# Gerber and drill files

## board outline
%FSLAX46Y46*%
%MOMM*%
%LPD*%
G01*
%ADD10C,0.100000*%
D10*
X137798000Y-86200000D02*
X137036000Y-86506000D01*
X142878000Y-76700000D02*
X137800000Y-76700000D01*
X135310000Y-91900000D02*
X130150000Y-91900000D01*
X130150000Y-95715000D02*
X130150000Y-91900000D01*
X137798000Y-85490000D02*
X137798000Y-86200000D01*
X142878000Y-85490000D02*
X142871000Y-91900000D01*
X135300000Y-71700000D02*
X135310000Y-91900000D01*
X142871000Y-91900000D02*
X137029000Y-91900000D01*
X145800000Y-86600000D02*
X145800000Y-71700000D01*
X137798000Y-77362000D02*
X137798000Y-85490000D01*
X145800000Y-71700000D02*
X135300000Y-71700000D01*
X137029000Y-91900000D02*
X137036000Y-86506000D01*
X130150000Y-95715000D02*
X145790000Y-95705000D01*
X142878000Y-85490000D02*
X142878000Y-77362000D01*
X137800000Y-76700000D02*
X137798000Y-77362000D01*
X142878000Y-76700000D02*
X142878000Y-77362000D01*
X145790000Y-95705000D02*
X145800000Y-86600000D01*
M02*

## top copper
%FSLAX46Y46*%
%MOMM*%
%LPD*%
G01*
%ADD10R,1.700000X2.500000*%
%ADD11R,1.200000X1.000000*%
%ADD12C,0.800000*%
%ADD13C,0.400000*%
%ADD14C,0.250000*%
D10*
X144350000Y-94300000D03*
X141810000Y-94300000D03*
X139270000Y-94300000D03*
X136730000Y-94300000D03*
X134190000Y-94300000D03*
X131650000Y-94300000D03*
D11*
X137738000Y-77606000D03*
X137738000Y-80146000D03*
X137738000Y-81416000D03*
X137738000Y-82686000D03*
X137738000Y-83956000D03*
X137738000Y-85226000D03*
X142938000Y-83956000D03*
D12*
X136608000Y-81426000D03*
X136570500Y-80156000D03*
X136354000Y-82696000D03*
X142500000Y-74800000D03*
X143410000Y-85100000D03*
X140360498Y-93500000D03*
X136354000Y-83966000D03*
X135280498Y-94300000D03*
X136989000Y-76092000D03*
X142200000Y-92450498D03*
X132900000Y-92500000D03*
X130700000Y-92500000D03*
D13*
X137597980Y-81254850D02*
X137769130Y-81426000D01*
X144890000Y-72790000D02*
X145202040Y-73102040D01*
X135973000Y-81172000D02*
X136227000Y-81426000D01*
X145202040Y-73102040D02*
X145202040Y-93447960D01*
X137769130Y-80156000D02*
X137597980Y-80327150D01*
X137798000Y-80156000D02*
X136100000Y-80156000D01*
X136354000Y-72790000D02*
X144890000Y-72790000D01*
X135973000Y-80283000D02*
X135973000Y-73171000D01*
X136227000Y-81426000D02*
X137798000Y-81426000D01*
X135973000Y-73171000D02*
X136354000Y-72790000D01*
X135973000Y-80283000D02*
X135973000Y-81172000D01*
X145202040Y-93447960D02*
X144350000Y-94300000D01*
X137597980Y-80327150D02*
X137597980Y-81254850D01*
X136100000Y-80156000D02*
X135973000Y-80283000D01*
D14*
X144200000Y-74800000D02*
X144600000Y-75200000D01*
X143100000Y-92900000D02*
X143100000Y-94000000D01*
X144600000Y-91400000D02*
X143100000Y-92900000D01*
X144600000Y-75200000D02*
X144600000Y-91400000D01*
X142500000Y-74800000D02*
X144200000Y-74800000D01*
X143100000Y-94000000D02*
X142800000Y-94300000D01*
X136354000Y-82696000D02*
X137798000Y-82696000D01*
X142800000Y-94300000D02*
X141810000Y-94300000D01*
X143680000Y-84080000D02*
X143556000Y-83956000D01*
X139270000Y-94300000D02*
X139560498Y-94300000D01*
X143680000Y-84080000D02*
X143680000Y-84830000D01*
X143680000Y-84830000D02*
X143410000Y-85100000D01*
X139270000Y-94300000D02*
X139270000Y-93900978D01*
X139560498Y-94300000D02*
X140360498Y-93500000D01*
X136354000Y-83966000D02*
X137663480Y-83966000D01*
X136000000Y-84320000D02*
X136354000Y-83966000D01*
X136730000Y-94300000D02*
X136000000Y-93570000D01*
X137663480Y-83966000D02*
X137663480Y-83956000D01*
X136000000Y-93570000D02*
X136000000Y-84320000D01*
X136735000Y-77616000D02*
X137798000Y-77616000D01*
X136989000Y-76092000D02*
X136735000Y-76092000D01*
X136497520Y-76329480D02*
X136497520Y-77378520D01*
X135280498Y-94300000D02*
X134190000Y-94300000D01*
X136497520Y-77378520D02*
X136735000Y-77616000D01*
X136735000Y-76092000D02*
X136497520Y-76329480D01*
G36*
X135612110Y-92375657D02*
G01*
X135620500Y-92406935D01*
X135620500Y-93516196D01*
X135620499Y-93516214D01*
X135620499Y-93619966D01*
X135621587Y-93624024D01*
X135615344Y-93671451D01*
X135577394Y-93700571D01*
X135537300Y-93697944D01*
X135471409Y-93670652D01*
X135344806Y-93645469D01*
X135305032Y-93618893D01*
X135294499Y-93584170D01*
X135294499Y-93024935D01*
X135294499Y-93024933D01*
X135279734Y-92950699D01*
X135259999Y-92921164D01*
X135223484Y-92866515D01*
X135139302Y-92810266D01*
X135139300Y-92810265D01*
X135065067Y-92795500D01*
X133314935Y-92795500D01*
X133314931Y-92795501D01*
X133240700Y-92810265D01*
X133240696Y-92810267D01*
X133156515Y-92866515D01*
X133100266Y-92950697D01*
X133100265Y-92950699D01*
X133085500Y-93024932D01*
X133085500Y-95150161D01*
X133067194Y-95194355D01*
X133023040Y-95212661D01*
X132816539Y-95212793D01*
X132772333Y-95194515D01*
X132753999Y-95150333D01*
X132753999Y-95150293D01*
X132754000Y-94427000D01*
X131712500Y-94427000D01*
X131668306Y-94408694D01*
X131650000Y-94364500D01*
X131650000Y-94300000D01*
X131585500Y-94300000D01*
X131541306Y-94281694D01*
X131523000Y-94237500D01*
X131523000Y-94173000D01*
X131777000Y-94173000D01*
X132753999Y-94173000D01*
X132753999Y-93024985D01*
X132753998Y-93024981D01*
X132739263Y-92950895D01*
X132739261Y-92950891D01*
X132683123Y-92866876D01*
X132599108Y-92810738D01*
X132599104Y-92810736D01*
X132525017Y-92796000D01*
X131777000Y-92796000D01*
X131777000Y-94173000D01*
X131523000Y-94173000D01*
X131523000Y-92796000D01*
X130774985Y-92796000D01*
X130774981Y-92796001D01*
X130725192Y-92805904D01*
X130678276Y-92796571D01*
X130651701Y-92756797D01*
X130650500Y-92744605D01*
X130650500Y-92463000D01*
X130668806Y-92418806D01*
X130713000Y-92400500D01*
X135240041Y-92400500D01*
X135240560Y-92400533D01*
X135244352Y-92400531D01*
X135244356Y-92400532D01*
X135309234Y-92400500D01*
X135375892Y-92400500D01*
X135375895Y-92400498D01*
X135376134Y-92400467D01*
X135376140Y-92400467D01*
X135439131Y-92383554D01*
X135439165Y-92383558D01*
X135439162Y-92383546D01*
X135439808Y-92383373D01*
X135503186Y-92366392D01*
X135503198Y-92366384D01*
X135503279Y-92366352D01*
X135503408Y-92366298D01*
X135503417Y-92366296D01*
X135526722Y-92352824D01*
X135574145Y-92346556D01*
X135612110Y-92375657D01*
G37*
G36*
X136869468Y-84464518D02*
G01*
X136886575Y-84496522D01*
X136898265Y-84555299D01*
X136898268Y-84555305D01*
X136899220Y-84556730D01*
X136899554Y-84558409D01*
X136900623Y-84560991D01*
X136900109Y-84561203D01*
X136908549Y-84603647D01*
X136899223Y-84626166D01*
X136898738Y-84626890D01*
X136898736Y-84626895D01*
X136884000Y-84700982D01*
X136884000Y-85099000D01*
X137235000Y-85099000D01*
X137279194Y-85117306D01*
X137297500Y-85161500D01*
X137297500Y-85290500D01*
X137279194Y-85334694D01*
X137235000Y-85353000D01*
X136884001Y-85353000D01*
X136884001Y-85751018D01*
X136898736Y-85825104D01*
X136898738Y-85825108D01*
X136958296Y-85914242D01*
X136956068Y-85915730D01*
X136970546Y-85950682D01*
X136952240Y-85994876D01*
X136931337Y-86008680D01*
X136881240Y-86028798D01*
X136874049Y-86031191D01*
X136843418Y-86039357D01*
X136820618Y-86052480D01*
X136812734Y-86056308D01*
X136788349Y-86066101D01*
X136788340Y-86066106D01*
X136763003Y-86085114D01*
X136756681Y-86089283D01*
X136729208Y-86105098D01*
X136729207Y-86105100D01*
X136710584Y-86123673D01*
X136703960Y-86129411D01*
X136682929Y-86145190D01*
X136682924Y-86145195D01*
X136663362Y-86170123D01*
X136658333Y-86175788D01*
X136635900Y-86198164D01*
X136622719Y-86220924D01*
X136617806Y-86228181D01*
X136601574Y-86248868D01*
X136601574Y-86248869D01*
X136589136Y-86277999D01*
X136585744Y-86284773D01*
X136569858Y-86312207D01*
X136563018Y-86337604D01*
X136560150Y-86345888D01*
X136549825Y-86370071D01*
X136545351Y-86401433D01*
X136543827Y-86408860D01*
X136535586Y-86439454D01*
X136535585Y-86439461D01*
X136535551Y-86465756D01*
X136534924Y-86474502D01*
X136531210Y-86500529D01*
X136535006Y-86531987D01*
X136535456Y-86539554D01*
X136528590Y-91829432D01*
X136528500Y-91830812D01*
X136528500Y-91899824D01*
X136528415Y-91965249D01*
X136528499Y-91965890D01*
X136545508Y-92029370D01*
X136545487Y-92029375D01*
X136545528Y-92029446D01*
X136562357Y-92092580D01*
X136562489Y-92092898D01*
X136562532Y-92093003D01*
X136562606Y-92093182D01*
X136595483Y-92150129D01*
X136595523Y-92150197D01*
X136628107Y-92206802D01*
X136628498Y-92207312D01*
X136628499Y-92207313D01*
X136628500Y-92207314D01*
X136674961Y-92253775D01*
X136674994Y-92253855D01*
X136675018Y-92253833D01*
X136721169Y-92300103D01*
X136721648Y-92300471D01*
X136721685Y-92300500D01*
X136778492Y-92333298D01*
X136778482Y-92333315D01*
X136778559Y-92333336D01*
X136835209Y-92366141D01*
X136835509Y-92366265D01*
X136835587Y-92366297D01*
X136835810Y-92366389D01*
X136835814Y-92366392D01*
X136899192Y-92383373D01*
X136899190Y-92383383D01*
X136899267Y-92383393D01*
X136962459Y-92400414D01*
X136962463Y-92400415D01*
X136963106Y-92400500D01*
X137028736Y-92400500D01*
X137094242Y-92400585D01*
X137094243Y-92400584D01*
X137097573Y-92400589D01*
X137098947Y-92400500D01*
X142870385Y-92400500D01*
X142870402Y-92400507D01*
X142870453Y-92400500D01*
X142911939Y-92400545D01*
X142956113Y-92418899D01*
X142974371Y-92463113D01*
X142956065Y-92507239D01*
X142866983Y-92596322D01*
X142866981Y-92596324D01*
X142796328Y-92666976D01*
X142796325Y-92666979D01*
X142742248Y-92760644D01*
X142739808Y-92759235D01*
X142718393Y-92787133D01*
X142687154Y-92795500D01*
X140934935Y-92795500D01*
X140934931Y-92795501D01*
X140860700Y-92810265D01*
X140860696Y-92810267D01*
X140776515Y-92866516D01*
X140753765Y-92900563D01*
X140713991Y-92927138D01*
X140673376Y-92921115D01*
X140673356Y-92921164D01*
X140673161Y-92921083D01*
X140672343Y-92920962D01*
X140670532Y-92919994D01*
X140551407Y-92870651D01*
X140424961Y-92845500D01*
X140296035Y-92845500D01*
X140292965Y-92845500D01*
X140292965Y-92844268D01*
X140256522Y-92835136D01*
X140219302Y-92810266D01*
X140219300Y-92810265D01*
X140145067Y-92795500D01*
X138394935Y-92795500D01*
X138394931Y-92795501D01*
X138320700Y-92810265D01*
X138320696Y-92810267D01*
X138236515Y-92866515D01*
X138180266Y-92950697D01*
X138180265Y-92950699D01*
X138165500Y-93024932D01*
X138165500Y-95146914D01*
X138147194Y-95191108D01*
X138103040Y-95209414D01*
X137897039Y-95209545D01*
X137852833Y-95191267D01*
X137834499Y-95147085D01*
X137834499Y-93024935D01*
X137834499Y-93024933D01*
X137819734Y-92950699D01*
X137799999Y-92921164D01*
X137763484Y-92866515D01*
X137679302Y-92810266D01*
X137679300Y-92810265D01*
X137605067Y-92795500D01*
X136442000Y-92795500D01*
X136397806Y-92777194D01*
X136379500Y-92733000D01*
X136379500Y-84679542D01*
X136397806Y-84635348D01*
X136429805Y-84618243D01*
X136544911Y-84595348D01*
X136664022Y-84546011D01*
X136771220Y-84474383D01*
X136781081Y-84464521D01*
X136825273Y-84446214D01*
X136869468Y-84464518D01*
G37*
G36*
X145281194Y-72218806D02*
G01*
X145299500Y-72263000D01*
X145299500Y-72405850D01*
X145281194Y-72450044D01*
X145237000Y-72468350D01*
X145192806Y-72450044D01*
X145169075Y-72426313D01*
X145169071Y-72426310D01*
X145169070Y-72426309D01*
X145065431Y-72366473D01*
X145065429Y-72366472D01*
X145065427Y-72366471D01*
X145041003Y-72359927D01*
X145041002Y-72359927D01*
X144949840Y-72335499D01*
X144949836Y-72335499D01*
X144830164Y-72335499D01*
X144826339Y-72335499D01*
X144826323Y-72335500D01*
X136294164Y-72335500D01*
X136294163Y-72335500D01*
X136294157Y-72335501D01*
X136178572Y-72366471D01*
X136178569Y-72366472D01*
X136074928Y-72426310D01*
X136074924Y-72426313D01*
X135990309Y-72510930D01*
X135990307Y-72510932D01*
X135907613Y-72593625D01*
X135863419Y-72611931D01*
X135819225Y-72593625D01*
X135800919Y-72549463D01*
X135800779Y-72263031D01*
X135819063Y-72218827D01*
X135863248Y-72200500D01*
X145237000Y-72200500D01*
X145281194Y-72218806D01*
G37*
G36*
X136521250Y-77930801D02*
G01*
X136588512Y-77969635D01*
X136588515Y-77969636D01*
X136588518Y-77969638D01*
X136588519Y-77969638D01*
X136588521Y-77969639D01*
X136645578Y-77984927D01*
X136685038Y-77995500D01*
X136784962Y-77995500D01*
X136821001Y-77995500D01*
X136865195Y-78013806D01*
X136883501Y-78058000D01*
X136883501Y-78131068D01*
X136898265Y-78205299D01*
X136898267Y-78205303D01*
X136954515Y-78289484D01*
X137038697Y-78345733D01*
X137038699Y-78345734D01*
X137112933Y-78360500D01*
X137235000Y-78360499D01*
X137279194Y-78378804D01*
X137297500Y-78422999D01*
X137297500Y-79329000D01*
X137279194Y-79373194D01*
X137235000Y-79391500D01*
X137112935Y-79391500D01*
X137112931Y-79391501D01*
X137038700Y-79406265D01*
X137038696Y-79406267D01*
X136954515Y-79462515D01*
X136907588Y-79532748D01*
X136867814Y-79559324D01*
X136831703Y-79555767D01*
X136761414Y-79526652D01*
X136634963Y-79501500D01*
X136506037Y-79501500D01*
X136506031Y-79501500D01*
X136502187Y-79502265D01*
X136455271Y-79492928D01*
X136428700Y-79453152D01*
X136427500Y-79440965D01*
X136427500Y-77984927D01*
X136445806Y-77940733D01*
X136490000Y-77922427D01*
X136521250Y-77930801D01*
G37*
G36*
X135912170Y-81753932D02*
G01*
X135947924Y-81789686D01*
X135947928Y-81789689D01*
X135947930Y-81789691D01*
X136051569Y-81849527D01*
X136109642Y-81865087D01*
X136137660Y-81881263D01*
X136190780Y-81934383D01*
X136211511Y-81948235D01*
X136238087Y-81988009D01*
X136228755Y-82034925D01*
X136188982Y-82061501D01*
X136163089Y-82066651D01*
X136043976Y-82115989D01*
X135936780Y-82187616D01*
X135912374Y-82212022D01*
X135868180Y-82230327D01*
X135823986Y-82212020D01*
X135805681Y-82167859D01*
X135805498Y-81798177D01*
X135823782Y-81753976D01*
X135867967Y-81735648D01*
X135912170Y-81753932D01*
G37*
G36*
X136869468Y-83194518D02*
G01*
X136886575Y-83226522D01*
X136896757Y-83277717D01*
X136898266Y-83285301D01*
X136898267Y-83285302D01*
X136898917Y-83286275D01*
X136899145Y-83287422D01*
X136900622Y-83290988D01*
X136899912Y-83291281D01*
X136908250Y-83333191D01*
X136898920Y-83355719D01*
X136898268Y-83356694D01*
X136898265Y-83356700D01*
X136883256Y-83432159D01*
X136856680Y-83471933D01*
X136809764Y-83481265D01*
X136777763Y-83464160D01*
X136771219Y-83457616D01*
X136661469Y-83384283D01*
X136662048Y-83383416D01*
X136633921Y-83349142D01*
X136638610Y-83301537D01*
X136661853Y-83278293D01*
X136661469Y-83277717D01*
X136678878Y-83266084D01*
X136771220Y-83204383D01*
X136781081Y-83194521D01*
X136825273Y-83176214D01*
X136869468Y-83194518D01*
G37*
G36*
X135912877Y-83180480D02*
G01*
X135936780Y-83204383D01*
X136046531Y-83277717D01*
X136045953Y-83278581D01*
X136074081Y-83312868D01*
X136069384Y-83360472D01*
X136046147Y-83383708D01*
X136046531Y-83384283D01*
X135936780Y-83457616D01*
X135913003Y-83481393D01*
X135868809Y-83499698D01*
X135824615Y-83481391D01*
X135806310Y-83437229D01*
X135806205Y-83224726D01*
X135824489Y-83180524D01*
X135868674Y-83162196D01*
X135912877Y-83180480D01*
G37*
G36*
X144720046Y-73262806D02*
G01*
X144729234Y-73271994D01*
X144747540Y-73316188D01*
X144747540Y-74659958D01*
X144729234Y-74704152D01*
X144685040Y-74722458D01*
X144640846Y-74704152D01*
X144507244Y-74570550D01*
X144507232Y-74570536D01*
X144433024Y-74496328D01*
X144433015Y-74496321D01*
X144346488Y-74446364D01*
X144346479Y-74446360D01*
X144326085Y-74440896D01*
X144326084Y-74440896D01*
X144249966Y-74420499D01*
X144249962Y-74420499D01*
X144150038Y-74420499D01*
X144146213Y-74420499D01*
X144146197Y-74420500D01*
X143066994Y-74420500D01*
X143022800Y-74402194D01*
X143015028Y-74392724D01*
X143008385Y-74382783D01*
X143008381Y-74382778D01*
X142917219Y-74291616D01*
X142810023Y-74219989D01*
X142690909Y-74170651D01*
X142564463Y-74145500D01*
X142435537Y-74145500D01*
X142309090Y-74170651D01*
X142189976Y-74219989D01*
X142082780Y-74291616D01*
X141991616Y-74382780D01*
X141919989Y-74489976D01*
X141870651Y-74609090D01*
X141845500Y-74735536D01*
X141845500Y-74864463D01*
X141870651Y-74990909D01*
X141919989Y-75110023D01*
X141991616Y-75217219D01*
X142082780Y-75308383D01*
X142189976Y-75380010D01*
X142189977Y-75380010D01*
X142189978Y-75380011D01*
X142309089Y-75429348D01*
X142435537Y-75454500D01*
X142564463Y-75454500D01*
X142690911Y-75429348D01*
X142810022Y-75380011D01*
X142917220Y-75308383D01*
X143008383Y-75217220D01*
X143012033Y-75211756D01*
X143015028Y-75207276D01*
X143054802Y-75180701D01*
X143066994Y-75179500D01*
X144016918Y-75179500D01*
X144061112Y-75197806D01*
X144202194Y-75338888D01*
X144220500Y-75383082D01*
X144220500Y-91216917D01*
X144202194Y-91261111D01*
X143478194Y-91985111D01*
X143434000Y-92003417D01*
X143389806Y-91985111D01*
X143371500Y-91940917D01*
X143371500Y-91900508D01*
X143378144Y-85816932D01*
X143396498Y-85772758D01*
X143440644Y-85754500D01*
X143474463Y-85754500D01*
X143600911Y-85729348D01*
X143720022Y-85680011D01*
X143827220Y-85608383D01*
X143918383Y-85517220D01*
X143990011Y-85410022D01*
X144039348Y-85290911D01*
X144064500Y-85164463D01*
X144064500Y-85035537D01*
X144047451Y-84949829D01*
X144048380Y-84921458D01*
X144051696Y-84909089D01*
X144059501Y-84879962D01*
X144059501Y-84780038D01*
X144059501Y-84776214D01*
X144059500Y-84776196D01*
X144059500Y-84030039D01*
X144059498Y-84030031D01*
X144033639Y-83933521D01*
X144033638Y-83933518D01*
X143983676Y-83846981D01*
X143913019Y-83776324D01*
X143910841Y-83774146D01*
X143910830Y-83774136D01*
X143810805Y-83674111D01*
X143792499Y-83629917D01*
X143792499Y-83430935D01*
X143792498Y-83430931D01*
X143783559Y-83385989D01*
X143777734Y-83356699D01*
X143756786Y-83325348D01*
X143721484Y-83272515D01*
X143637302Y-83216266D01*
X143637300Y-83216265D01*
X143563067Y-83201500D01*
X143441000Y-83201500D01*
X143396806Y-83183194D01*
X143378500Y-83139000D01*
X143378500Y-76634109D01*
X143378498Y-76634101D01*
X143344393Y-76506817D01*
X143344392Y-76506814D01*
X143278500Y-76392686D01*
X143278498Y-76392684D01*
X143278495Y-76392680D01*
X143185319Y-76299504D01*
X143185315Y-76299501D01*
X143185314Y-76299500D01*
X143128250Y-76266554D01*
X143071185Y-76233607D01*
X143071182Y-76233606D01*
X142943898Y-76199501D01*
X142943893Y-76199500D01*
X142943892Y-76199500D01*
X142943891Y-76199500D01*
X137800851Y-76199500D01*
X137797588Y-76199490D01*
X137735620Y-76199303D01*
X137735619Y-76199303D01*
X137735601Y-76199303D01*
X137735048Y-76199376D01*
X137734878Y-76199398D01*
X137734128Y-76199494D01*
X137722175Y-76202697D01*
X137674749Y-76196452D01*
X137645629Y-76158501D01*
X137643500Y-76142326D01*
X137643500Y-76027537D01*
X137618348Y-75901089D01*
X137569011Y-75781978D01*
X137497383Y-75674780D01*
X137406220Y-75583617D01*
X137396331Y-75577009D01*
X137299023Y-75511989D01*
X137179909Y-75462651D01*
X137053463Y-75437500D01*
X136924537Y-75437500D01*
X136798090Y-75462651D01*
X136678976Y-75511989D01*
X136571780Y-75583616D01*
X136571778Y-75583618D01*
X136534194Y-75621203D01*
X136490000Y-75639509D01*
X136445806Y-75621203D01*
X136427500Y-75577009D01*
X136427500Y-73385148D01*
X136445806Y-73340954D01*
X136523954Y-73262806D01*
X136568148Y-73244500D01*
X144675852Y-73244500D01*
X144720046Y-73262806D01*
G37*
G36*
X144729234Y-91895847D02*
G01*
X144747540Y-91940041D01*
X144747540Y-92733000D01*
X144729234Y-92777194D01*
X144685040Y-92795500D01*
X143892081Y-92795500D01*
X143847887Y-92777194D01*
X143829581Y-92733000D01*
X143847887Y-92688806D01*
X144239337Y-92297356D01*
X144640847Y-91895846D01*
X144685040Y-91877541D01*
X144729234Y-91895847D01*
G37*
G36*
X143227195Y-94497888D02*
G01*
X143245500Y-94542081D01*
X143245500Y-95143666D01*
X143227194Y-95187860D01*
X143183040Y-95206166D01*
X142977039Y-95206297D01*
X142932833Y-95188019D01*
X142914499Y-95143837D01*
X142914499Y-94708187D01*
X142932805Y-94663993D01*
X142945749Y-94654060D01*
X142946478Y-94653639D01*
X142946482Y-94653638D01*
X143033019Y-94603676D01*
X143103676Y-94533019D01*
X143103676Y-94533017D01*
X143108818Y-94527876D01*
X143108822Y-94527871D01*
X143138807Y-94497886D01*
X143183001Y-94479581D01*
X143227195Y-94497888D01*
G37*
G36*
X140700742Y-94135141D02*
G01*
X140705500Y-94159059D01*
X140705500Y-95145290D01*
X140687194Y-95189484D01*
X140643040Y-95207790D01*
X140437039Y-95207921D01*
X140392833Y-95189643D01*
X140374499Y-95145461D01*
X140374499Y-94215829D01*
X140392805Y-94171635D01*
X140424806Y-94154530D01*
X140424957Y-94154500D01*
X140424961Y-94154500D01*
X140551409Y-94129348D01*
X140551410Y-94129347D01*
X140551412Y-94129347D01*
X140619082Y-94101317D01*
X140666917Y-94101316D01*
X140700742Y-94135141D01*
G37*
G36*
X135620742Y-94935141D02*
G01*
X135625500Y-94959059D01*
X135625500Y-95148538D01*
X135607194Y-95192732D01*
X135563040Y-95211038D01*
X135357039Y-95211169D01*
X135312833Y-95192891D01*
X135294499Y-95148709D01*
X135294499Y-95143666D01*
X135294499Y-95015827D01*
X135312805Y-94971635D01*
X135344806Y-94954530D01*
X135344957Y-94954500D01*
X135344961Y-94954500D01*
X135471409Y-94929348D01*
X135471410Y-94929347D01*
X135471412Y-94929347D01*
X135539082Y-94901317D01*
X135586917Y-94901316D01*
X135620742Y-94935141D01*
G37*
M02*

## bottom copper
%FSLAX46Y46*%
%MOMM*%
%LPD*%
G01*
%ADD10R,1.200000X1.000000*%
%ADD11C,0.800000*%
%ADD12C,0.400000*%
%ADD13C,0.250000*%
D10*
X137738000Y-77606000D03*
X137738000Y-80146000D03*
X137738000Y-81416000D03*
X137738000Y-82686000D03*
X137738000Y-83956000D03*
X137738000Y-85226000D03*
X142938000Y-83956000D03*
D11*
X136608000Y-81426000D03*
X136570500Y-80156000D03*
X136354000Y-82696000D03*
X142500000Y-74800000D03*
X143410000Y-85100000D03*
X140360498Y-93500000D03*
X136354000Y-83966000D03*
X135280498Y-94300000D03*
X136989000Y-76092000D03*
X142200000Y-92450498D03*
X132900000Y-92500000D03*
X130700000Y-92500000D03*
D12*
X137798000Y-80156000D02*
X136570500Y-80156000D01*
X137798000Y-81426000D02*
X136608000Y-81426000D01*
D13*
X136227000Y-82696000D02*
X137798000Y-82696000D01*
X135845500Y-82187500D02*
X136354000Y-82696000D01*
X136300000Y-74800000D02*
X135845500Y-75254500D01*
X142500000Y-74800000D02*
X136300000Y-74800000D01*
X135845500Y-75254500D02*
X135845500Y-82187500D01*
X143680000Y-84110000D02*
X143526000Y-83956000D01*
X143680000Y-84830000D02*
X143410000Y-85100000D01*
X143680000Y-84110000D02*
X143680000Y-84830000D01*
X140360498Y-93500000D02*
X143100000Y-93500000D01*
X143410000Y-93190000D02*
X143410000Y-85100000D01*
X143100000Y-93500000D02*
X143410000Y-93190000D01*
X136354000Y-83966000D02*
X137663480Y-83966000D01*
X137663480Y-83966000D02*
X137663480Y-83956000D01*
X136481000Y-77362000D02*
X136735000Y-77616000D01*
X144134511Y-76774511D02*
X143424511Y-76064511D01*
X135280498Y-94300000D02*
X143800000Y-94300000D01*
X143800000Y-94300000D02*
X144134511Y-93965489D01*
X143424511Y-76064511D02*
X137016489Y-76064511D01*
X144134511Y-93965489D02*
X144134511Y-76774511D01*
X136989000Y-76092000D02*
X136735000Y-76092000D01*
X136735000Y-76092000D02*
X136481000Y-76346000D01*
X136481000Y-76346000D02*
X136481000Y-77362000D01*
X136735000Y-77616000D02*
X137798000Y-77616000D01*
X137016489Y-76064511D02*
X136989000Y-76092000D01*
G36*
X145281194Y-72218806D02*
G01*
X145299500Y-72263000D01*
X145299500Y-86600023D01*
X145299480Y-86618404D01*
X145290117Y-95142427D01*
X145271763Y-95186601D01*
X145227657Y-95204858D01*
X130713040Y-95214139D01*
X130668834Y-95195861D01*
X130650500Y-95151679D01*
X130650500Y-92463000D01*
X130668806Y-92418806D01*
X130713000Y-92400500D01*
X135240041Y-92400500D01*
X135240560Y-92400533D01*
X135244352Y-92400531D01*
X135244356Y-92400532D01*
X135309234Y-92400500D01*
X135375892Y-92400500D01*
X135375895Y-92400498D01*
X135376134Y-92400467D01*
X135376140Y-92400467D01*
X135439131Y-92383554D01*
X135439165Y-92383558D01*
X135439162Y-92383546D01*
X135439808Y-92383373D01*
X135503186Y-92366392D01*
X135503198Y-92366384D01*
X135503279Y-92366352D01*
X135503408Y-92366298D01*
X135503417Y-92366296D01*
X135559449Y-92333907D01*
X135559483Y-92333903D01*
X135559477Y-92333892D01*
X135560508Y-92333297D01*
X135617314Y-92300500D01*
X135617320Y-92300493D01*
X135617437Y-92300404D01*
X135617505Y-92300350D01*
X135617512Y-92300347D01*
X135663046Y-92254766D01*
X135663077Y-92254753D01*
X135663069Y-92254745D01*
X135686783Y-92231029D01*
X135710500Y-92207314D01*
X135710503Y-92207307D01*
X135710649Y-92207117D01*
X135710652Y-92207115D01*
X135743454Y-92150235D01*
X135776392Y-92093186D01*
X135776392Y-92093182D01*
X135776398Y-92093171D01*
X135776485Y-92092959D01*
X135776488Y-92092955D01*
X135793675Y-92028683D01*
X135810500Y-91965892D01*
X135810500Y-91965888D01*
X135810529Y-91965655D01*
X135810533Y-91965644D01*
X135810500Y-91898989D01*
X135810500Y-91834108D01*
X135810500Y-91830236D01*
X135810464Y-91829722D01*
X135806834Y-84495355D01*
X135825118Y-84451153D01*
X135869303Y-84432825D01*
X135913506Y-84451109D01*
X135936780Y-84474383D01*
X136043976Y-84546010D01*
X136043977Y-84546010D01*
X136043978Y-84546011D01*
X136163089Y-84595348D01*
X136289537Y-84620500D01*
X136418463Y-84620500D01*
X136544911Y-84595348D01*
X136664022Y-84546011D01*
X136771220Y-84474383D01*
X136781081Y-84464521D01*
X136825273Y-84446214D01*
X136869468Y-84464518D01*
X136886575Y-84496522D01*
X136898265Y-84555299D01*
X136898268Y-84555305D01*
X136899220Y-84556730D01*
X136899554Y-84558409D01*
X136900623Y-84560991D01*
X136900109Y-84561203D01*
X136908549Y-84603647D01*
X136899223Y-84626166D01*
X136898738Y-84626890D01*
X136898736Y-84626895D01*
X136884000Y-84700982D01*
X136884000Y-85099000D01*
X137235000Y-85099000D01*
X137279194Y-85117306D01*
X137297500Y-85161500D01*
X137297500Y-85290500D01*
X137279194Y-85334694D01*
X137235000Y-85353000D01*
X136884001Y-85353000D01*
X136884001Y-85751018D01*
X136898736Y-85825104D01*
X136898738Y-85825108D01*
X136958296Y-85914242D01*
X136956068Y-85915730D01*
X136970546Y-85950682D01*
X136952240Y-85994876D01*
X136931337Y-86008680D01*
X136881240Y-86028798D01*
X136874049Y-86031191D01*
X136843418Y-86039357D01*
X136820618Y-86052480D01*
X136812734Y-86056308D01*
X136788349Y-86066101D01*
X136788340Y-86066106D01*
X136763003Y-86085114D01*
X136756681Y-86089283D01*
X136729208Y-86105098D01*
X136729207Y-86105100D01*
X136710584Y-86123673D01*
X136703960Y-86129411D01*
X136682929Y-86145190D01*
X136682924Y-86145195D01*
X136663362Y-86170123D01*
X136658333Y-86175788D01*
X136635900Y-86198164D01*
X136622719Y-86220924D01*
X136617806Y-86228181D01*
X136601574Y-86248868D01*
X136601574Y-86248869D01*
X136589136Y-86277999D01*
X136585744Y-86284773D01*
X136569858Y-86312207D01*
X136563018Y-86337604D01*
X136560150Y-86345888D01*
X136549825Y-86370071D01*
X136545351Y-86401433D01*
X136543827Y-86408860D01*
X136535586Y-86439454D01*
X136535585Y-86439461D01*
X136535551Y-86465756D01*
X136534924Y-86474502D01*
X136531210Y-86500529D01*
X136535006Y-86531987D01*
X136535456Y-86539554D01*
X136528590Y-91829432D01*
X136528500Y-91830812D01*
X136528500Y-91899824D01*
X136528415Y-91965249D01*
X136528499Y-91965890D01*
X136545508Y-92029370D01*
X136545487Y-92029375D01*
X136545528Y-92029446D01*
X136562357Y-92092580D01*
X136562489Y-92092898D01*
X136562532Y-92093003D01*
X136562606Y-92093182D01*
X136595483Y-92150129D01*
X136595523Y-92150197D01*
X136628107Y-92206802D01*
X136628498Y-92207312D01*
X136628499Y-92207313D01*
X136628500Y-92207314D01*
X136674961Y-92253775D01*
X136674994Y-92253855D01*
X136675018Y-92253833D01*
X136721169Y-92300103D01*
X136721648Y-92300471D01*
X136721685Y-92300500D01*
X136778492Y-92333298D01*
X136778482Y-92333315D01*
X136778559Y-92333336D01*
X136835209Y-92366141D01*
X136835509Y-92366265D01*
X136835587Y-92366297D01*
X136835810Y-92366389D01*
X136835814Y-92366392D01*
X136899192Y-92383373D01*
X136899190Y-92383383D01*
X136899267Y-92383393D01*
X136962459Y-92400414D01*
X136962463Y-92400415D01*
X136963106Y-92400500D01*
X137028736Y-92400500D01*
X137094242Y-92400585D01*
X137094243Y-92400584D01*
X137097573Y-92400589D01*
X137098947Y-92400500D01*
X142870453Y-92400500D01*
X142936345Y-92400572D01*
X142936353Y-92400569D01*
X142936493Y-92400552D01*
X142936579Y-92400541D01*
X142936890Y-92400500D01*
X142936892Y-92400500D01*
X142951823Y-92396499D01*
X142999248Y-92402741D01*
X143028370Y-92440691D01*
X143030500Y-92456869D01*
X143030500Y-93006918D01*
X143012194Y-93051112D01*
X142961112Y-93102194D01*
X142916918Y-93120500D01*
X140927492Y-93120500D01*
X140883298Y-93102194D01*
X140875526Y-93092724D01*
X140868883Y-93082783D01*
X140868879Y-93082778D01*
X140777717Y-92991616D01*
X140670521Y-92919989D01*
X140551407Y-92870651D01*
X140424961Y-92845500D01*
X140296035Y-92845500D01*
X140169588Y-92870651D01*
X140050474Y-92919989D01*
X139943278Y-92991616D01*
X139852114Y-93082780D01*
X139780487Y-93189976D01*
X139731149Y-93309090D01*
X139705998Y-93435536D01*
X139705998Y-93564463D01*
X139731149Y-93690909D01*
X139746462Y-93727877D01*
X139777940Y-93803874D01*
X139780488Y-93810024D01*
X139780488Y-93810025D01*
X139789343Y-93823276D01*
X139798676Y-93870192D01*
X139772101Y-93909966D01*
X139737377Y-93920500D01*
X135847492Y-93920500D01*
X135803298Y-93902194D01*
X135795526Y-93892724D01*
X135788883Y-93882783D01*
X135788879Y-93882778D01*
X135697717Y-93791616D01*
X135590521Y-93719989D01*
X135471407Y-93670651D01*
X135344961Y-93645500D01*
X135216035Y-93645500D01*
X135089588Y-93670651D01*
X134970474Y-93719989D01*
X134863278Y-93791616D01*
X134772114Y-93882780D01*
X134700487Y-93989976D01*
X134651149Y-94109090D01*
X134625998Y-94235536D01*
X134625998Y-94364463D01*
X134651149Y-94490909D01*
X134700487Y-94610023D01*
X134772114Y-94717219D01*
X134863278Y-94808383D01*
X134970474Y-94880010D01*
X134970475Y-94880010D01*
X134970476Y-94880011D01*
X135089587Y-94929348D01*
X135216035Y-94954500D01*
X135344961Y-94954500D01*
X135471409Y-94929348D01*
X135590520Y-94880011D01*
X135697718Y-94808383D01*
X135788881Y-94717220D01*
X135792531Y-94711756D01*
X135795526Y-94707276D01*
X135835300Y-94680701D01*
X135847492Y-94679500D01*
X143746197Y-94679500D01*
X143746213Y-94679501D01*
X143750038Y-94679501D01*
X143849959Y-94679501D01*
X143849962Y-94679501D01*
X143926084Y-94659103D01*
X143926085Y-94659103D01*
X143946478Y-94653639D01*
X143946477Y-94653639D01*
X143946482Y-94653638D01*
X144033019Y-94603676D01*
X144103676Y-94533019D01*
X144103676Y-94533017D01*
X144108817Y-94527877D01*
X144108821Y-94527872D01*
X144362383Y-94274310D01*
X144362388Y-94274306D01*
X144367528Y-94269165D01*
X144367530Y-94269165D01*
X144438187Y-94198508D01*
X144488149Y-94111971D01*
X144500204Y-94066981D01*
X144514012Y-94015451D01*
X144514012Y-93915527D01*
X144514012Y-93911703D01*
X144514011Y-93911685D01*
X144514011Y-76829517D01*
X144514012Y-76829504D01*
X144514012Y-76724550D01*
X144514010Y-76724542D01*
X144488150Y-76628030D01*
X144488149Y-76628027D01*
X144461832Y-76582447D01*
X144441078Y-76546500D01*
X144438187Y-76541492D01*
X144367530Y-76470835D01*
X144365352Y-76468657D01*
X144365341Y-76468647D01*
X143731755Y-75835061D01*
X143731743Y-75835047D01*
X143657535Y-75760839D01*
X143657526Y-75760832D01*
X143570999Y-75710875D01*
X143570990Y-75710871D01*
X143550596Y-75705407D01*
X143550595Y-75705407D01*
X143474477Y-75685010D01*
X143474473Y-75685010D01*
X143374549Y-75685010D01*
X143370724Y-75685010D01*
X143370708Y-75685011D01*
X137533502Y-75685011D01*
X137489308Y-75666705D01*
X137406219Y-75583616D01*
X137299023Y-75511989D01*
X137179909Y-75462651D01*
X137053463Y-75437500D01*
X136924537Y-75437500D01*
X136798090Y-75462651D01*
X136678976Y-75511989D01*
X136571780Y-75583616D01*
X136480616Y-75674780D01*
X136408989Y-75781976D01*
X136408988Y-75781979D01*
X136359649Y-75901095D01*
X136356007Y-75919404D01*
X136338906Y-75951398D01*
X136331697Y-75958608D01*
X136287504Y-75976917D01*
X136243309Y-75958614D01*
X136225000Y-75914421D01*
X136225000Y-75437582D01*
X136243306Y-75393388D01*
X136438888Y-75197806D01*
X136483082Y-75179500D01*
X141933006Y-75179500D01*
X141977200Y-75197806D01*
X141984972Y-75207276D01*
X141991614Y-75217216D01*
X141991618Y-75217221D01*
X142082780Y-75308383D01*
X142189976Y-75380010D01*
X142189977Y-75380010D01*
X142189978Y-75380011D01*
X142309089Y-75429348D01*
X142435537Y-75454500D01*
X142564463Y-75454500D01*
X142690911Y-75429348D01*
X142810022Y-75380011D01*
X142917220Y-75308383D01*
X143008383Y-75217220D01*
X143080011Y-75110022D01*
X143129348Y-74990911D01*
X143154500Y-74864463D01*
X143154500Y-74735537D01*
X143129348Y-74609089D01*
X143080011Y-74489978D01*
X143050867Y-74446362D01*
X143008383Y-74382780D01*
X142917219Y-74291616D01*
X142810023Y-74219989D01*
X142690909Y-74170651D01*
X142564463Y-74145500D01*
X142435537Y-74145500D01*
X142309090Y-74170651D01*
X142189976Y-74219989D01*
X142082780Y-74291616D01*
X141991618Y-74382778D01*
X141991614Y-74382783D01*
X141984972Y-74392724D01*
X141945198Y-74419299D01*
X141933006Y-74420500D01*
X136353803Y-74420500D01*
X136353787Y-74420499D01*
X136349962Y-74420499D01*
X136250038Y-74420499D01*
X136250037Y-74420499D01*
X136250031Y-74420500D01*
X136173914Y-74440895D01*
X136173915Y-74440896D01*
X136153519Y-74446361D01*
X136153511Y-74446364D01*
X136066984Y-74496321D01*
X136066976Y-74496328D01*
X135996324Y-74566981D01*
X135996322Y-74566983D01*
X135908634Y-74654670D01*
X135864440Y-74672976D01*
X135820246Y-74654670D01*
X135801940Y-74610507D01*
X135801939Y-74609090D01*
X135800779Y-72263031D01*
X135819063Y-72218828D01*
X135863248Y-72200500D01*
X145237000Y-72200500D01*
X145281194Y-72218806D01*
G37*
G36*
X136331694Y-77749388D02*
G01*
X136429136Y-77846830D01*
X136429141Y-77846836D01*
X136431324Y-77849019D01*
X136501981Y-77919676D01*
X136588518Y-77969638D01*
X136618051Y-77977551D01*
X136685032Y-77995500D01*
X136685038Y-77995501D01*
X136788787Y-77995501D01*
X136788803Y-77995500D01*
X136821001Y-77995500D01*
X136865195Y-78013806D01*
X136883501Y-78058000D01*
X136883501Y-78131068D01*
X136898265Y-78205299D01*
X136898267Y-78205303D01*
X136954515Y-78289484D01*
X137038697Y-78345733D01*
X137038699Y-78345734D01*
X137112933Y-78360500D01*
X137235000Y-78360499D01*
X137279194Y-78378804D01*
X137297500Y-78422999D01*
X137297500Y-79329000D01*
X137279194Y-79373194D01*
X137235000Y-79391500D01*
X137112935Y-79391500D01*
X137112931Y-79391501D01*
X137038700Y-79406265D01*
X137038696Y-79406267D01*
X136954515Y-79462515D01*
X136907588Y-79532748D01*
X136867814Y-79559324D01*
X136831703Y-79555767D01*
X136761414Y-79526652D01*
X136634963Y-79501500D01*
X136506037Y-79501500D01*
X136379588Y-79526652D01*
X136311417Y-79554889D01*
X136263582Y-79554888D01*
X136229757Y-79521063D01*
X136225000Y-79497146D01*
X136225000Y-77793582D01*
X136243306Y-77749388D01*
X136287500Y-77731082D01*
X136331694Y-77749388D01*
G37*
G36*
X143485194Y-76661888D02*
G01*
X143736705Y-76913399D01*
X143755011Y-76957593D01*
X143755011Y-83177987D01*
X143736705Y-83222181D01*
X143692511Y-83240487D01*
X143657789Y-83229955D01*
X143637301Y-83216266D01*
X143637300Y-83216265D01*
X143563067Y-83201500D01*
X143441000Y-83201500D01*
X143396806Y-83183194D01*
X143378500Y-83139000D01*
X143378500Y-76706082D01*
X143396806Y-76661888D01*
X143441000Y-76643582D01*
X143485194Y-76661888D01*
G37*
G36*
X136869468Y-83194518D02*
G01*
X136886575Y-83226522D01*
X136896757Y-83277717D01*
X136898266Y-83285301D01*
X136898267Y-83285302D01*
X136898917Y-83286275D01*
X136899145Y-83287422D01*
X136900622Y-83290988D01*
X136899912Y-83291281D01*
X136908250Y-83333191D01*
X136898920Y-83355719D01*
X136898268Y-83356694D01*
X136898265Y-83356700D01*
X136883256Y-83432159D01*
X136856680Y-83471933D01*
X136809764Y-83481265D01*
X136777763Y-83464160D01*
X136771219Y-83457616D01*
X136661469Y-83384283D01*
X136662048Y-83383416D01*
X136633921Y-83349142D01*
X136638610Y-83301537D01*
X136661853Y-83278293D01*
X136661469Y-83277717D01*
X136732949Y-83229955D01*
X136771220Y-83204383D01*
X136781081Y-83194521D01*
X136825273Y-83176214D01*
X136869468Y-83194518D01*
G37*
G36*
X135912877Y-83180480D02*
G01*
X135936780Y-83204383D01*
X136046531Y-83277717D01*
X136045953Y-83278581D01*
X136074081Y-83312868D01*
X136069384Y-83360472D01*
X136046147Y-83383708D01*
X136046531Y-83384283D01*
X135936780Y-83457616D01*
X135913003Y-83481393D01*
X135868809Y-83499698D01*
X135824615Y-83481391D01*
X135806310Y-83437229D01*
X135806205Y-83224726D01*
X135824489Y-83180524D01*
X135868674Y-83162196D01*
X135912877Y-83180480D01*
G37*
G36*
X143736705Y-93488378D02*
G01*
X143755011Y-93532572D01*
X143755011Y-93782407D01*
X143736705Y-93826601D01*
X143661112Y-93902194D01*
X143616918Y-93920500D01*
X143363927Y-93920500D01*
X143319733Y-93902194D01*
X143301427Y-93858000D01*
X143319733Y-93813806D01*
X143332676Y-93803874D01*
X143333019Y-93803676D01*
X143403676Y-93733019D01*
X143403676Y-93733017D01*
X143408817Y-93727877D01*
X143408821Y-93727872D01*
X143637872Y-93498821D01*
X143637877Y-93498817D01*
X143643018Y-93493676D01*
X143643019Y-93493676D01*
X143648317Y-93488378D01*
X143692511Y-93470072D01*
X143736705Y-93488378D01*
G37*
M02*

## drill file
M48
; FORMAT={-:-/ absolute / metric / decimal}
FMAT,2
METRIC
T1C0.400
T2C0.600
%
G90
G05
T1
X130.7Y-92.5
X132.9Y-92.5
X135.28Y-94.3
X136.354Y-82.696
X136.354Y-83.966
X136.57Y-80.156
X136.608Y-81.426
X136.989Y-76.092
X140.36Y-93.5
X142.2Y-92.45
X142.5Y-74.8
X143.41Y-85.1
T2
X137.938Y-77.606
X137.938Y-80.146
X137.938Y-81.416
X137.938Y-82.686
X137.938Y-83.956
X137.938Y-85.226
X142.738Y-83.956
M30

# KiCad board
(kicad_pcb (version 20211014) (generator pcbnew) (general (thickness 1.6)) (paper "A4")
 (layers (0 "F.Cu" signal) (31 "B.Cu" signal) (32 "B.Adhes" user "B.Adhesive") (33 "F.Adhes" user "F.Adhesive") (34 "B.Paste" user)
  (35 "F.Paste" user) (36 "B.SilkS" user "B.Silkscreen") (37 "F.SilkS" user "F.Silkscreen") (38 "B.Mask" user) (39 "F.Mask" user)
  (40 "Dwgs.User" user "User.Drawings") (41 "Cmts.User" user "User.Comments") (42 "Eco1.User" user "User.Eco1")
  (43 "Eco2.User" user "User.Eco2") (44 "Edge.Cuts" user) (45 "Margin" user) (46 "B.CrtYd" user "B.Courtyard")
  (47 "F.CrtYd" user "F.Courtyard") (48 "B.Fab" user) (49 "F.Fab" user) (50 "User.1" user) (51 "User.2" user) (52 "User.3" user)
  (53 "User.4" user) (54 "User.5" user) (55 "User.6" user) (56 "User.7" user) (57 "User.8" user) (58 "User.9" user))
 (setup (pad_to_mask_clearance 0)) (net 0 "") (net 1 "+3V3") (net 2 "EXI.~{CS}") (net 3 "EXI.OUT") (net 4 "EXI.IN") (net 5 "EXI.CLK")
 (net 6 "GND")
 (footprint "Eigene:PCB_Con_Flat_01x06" (layer "F.Cu") (at 138 94.3 -90)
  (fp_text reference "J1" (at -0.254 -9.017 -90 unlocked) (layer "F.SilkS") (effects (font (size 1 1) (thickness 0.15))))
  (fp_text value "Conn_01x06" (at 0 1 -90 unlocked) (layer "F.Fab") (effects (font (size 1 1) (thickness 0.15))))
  (pad "1" smd rect (at 0 -6.35 270) (size 2.5 1.7) (layers "F.Cu" "F.Paste" "F.Mask") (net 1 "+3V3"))
  (pad "2" smd rect (at 0 -3.81 270) (size 2.5 1.7) (layers "F.Cu" "F.Paste" "F.Mask") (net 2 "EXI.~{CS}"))
  (pad "3" smd rect (at 0 -1.27 270) (size 2.5 1.7) (layers "F.Cu" "F.Paste" "F.Mask") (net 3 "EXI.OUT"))
  (pad "4" smd rect (at 0 1.27 270) (size 2.5 1.7) (layers "F.Cu" "F.Paste" "F.Mask") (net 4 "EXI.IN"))
  (pad "5" smd rect (at 0 3.81 270) (size 2.5 1.7) (layers "F.Cu" "F.Paste" "F.Mask") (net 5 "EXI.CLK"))
  (pad "6" smd rect (at 0 6.35 270) (size 2.5 1.7) (layers "F.Cu" "F.Paste" "F.Mask") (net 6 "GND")))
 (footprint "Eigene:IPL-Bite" (layer "F.Cu") (at 140.338 81.426)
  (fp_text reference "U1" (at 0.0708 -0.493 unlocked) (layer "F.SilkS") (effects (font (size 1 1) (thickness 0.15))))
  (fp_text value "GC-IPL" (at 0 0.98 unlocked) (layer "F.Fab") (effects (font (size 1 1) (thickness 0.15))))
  (pad "1" thru_hole rect (at -2.4 -3.82) (size 1.2 1) (drill 0.6 (offset -0.2 0)) (layers *.Cu *.Mask) (remove_unused_layers)
   (keep_end_layers) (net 5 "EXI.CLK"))
  (pad "3" thru_hole rect (at -2.4 -1.28) (size 1.2 1) (drill 0.6 (offset -0.2 0)) (layers *.Cu *.Mask) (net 1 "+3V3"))
  (pad "4" thru_hole rect (at -2.4 -0.01) (size 1.2 1) (drill 0.6 (offset -0.2 0)) (layers *.Cu *.Mask) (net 1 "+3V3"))
  (pad "5" thru_hole rect (at -2.4 1.26) (size 1.2 1) (drill 0.6 (offset -0.2 0)) (layers *.Cu *.Mask) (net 2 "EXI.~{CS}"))
  (pad "6" thru_hole rect (at -2.4 2.53) (size 1.2 1) (drill 0.6 (offset -0.2 0)) (layers *.Cu *.Mask) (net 4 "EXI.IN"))
  (pad "7" thru_hole rect (at -2.4 3.8) (size 1.2 1) (drill 0.6 (offset -0.2 0)) (layers *.Cu *.Mask) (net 6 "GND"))
  (pad "9" thru_hole rect (at 2.4 2.53 180) (size 1.2 1) (drill 0.6 (offset -0.2 0)) (layers *.Cu *.Mask) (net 3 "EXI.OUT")))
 (gr_line (start 137.798 86.2) (end 137.036 86.506) (layer "Edge.Cuts") (width 0.1))
 (gr_line (start 142.878 76.7) (end 137.8 76.7) (layer "Edge.Cuts") (width 0.1))
 (gr_line (start 135.31 91.9) (end 130.15 91.9) (layer "Edge.Cuts") (width 0.1))
 (gr_line (start 130.15 95.715) (end 130.15 91.9) (layer "Edge.Cuts") (width 0.1))
 (gr_line (start 137.798 85.49) (end 137.798 86.2) (layer "Edge.Cuts") (width 0.1))
 (gr_line (start 142.878 85.49) (end 142.871 91.9) (layer "Edge.Cuts") (width 0.1))
 (gr_line (start 135.3 71.7) (end 135.31 91.9) (layer "Edge.Cuts") (width 0.1))
 (gr_line (start 142.871 91.9) (end 137.029 91.9) (layer "Edge.Cuts") (width 0.1))
 (gr_line (start 145.8 86.6) (end 145.8 71.7) (layer "Edge.Cuts") (width 0.1))
 (gr_line (start 137.798 77.362) (end 137.798 85.49) (layer "Edge.Cuts") (width 0.1))
 (gr_line (start 145.8 71.7) (end 135.3 71.7) (layer "Edge.Cuts") (width 0.1))
 (gr_line (start 137.029 91.9) (end 137.036 86.506) (layer "Edge.Cuts") (width 0.1))
 (gr_line (start 130.15 95.715) (end 145.79 95.705) (layer "Edge.Cuts") (width 0.1))
 (gr_line (start 142.878 85.49) (end 142.878 77.362) (layer "Edge.Cuts") (width 0.1))
 (gr_line (start 137.8 76.7) (end 137.798 77.362) (layer "Edge.Cuts") (width 0.1))
 (gr_line (start 142.878 76.7) (end 142.878 77.362) (layer "Edge.Cuts") (width 0.1))
 (gr_line (start 145.79 95.705) (end 145.8 86.6) (layer "Edge.Cuts") (width 0.1))
 (segment (start 137.59798 81.25485) (end 137.76913 81.426) (width 0.4) (layer "F.Cu") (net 1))
 (segment (start 144.89 72.79) (end 145.20204 73.10204) (width 0.4) (layer "F.Cu") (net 1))
 (segment (start 135.973 81.172) (end 136.227 81.426) (width 0.4) (layer "F.Cu") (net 1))
 (segment (start 145.20204 73.10204) (end 145.20204 93.44796) (width 0.4) (layer "F.Cu") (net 1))
 (segment (start 137.76913 80.156) (end 137.59798 80.32715) (width 0.4) (layer "F.Cu") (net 1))
 (segment (start 137.798 80.156) (end 136.1 80.156) (width 0.4) (layer "F.Cu") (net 1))
 (segment (start 136.354 72.79) (end 144.89 72.79) (width 0.4) (layer "F.Cu") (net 1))
 (segment (start 135.973 80.283) (end 135.973 73.171) (width 0.4) (layer "F.Cu") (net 1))
 (segment (start 136.227 81.426) (end 137.798 81.426) (width 0.4) (layer "F.Cu") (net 1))
 (segment (start 135.973 73.171) (end 136.354 72.79) (width 0.4) (layer "F.Cu") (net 1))
 (segment (start 135.973 80.283) (end 135.973 81.172) (width 0.4) (layer "F.Cu") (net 1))
 (segment (start 145.20204 93.44796) (end 144.35 94.3) (width 0.4) (layer "F.Cu") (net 1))
 (segment (start 137.59798 80.32715) (end 137.59798 81.25485) (width 0.4) (layer "F.Cu") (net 1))
 (segment (start 136.1 80.156) (end 135.973 80.283) (width 0.4) (layer "F.Cu") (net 1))
 (via (at 136.608 81.426) (size 0.8) (drill 0.4) (layers "F.Cu" "B.Cu") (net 1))
 (via (at 136.5705 80.156) (size 0.8) (drill 0.4) (layers "F.Cu" "B.Cu") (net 1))
 (segment (start 137.798 80.156) (end 136.5705 80.156) (width 0.4) (layer "B.Cu") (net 1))
 (segment (start 137.798 81.426) (end 136.608 81.426) (width 0.4) (layer "B.Cu") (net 1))
 (segment (start 144.2 74.8) (end 144.6 75.2) (width 0.25) (layer "F.Cu") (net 2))
 (segment (start 143.1 92.9) (end 143.1 94) (width 0.25) (layer "F.Cu") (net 2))
 (segment (start 144.6 91.4) (end 143.1 92.9) (width 0.25) (layer "F.Cu") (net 2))
 (segment (start 144.6 75.2) (end 144.6 91.4) (width 0.25) (layer "F.Cu") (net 2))
 (segment (start 142.5 74.8) (end 144.2 74.8) (width 0.25) (layer "F.Cu") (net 2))
 (segment (start 143.1 94) (end 142.8 94.3) (width 0.25) (layer "F.Cu") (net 2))
 (segment (start 136.354 82.696) (end 137.798 82.696) (width 0.25) (layer "F.Cu") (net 2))
 (segment (start 142.8 94.3) (end 141.81 94.3) (width 0.25) (layer "F.Cu") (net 2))
 (via (at 136.354 82.696) (size 0.8) (drill 0.4) (layers "F.Cu" "B.Cu") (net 2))
 (via (at 142.5 74.8) (size 0.8) (drill 0.4) (layers "F.Cu" "B.Cu") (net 2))
 (segment (start 136.227 82.696) (end 137.798 82.696) (width 0.25) (layer "B.Cu") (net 2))
 (segment (start 135.8455 82.1875) (end 136.354 82.696) (width 0.25) (layer "B.Cu") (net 2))
 (segment (start 136.3 74.8) (end 135.8455 75.2545) (width 0.25) (layer "B.Cu") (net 2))
 (segment (start 142.5 74.8) (end 136.3 74.8) (width 0.25) (layer "B.Cu") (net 2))
 (segment (start 135.8455 75.2545) (end 135.8455 82.1875) (width 0.25) (layer "B.Cu") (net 2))
 (segment (start 143.68 84.08) (end 143.556 83.956) (width 0.25) (layer "F.Cu") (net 3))
 (segment (start 139.27 94.3) (end 139.560498 94.3) (width 0.25) (layer "F.Cu") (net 3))
 (segment (start 143.68 84.08) (end 143.68 84.83) (width 0.25) (layer "F.Cu") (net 3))
 (segment (start 143.68 84.83) (end 143.41 85.1) (width 0.25) (layer "F.Cu") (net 3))
 (segment (start 139.27 94.3) (end 139.27 93.900978) (width 0.25) (layer "F.Cu") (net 3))
 (segment (start 139.560498 94.3) (end 140.360498 93.5) (width 0.25) (layer "F.Cu") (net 3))
 (via (at 143.41 85.1) (size 0.8) (drill 0.4) (layers "F.Cu" "B.Cu") (free) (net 3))
 (via (at 140.360498 93.5) (size 0.8) (drill 0.4) (layers "F.Cu" "B.Cu") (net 3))
 (segment (start 143.68 84.11) (end 143.526 83.956) (width 0.25) (layer "B.Cu") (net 3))
 (segment (start 143.68 84.83) (end 143.41 85.1) (width 0.25) (layer "B.Cu") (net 3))
 (segment (start 143.68 84.11) (end 143.68 84.83) (width 0.25) (layer "B.Cu") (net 3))
 (segment (start 140.360498 93.5) (end 143.1 93.5) (width 0.25) (layer "B.Cu") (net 3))
 (segment (start 143.41 93.19) (end 143.41 85.1) (width 0.25) (layer "B.Cu") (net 3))
 (segment (start 143.1 93.5) (end 143.41 93.19) (width 0.25) (layer "B.Cu") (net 3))
 (segment (start 136.354 83.966) (end 137.66348 83.966) (width 0.25) (layer "F.Cu") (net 4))
 (segment (start 136 84.32) (end 136.354 83.966) (width 0.25) (layer "F.Cu") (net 4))
 (segment (start 136.73 94.3) (end 136 93.57) (width 0.25) (layer "F.Cu") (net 4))
 (segment (start 137.66348 83.966) (end 137.66348 83.956) (width 0.25) (layer "F.Cu") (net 4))
 (segment (start 136 93.57) (end 136 84.32) (width 0.25) (layer "F.Cu") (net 4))
 (via (at 136.354 83.966) (size 0.8) (drill 0.4) (layers "F.Cu" "B.Cu") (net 4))
 (segment (start 136.354 83.966) (end 137.66348 83.966) (width 0.25) (layer "B.Cu") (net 4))
 (segment (start 137.66348 83.966) (end 137.66348 83.956) (width 0.25) (layer "B.Cu") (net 4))
 (segment (start 136.735 77.616) (end 137.798 77.616) (width 0.25) (layer "F.Cu") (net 5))
 (segment (start 136.989 76.092) (end 136.735 76.092) (width 0.25) (layer "F.Cu") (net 5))
 (segment (start 136.49752 76.32948) (end 136.49752 77.37852) (width 0.25) (layer "F.Cu") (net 5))
 (segment (start 135.280498 94.3) (end 134.19 94.3) (width 0.25) (layer "F.Cu") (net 5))
 (segment (start 136.49752 77.37852) (end 136.735 77.616) (width 0.25) (layer "F.Cu") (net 5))
 (segment (start 136.735 76.092) (end 136.49752 76.32948) (width 0.25) (layer "F.Cu") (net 5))
 (via (at 135.280498 94.3) (size 0.8) (drill 0.4) (layers "F.Cu" "B.Cu") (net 5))
 (via (at 136.989 76.092) (size 0.8) (drill 0.4) (layers "F.Cu" "B.Cu") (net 5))
 (segment (start 136.481 77.362) (end 136.735 77.616) (width 0.25) (layer "B.Cu") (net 5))
 (segment (start 144.134511 76.774511) (end 143.424511 76.064511) (width 0.25) (layer "B.Cu") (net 5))
 (segment (start 135.280498 94.3) (end 143.8 94.3) (width 0.25) (layer "B.Cu") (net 5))
 (segment (start 143.8 94.3) (end 144.134511 93.965489) (width 0.25) (layer "B.Cu") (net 5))
 (segment (start 143.424511 76.064511) (end 137.016489 76.064511) (width 0.25) (layer "B.Cu") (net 5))
 (segment (start 144.134511 93.965489) (end 144.134511 76.774511) (width 0.25) (layer "B.Cu") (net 5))
 (segment (start 136.989 76.092) (end 136.735 76.092) (width 0.25) (layer "B.Cu") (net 5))
 (segment (start 136.735 76.092) (end 136.481 76.346) (width 0.25) (layer "B.Cu") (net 5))
 (segment (start 136.481 76.346) (end 136.481 77.362) (width 0.25) (layer "B.Cu") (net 5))
 (segment (start 136.735 77.616) (end 137.798 77.616) (width 0.25) (layer "B.Cu") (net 5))
 (segment (start 137.016489 76.064511) (end 136.989 76.092) (width 0.25) (layer "B.Cu") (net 5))
 (via (at 142.2 92.450498) (size 0.8) (drill 0.4) (layers "F.Cu" "B.Cu") (free) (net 6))
 (via (at 132.9 92.5) (size 0.8) (drill 0.4) (layers "F.Cu" "B.Cu") (free) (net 6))
 (via (at 130.7 92.5) (size 0.8) (drill 0.4) (layers "F.Cu" "B.Cu") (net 6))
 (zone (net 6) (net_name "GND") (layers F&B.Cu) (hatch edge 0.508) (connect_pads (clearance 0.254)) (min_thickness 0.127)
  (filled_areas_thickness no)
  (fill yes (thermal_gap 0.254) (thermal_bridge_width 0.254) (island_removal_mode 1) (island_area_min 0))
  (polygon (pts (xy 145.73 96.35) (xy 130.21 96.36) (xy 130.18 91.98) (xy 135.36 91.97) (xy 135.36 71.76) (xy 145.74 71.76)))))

